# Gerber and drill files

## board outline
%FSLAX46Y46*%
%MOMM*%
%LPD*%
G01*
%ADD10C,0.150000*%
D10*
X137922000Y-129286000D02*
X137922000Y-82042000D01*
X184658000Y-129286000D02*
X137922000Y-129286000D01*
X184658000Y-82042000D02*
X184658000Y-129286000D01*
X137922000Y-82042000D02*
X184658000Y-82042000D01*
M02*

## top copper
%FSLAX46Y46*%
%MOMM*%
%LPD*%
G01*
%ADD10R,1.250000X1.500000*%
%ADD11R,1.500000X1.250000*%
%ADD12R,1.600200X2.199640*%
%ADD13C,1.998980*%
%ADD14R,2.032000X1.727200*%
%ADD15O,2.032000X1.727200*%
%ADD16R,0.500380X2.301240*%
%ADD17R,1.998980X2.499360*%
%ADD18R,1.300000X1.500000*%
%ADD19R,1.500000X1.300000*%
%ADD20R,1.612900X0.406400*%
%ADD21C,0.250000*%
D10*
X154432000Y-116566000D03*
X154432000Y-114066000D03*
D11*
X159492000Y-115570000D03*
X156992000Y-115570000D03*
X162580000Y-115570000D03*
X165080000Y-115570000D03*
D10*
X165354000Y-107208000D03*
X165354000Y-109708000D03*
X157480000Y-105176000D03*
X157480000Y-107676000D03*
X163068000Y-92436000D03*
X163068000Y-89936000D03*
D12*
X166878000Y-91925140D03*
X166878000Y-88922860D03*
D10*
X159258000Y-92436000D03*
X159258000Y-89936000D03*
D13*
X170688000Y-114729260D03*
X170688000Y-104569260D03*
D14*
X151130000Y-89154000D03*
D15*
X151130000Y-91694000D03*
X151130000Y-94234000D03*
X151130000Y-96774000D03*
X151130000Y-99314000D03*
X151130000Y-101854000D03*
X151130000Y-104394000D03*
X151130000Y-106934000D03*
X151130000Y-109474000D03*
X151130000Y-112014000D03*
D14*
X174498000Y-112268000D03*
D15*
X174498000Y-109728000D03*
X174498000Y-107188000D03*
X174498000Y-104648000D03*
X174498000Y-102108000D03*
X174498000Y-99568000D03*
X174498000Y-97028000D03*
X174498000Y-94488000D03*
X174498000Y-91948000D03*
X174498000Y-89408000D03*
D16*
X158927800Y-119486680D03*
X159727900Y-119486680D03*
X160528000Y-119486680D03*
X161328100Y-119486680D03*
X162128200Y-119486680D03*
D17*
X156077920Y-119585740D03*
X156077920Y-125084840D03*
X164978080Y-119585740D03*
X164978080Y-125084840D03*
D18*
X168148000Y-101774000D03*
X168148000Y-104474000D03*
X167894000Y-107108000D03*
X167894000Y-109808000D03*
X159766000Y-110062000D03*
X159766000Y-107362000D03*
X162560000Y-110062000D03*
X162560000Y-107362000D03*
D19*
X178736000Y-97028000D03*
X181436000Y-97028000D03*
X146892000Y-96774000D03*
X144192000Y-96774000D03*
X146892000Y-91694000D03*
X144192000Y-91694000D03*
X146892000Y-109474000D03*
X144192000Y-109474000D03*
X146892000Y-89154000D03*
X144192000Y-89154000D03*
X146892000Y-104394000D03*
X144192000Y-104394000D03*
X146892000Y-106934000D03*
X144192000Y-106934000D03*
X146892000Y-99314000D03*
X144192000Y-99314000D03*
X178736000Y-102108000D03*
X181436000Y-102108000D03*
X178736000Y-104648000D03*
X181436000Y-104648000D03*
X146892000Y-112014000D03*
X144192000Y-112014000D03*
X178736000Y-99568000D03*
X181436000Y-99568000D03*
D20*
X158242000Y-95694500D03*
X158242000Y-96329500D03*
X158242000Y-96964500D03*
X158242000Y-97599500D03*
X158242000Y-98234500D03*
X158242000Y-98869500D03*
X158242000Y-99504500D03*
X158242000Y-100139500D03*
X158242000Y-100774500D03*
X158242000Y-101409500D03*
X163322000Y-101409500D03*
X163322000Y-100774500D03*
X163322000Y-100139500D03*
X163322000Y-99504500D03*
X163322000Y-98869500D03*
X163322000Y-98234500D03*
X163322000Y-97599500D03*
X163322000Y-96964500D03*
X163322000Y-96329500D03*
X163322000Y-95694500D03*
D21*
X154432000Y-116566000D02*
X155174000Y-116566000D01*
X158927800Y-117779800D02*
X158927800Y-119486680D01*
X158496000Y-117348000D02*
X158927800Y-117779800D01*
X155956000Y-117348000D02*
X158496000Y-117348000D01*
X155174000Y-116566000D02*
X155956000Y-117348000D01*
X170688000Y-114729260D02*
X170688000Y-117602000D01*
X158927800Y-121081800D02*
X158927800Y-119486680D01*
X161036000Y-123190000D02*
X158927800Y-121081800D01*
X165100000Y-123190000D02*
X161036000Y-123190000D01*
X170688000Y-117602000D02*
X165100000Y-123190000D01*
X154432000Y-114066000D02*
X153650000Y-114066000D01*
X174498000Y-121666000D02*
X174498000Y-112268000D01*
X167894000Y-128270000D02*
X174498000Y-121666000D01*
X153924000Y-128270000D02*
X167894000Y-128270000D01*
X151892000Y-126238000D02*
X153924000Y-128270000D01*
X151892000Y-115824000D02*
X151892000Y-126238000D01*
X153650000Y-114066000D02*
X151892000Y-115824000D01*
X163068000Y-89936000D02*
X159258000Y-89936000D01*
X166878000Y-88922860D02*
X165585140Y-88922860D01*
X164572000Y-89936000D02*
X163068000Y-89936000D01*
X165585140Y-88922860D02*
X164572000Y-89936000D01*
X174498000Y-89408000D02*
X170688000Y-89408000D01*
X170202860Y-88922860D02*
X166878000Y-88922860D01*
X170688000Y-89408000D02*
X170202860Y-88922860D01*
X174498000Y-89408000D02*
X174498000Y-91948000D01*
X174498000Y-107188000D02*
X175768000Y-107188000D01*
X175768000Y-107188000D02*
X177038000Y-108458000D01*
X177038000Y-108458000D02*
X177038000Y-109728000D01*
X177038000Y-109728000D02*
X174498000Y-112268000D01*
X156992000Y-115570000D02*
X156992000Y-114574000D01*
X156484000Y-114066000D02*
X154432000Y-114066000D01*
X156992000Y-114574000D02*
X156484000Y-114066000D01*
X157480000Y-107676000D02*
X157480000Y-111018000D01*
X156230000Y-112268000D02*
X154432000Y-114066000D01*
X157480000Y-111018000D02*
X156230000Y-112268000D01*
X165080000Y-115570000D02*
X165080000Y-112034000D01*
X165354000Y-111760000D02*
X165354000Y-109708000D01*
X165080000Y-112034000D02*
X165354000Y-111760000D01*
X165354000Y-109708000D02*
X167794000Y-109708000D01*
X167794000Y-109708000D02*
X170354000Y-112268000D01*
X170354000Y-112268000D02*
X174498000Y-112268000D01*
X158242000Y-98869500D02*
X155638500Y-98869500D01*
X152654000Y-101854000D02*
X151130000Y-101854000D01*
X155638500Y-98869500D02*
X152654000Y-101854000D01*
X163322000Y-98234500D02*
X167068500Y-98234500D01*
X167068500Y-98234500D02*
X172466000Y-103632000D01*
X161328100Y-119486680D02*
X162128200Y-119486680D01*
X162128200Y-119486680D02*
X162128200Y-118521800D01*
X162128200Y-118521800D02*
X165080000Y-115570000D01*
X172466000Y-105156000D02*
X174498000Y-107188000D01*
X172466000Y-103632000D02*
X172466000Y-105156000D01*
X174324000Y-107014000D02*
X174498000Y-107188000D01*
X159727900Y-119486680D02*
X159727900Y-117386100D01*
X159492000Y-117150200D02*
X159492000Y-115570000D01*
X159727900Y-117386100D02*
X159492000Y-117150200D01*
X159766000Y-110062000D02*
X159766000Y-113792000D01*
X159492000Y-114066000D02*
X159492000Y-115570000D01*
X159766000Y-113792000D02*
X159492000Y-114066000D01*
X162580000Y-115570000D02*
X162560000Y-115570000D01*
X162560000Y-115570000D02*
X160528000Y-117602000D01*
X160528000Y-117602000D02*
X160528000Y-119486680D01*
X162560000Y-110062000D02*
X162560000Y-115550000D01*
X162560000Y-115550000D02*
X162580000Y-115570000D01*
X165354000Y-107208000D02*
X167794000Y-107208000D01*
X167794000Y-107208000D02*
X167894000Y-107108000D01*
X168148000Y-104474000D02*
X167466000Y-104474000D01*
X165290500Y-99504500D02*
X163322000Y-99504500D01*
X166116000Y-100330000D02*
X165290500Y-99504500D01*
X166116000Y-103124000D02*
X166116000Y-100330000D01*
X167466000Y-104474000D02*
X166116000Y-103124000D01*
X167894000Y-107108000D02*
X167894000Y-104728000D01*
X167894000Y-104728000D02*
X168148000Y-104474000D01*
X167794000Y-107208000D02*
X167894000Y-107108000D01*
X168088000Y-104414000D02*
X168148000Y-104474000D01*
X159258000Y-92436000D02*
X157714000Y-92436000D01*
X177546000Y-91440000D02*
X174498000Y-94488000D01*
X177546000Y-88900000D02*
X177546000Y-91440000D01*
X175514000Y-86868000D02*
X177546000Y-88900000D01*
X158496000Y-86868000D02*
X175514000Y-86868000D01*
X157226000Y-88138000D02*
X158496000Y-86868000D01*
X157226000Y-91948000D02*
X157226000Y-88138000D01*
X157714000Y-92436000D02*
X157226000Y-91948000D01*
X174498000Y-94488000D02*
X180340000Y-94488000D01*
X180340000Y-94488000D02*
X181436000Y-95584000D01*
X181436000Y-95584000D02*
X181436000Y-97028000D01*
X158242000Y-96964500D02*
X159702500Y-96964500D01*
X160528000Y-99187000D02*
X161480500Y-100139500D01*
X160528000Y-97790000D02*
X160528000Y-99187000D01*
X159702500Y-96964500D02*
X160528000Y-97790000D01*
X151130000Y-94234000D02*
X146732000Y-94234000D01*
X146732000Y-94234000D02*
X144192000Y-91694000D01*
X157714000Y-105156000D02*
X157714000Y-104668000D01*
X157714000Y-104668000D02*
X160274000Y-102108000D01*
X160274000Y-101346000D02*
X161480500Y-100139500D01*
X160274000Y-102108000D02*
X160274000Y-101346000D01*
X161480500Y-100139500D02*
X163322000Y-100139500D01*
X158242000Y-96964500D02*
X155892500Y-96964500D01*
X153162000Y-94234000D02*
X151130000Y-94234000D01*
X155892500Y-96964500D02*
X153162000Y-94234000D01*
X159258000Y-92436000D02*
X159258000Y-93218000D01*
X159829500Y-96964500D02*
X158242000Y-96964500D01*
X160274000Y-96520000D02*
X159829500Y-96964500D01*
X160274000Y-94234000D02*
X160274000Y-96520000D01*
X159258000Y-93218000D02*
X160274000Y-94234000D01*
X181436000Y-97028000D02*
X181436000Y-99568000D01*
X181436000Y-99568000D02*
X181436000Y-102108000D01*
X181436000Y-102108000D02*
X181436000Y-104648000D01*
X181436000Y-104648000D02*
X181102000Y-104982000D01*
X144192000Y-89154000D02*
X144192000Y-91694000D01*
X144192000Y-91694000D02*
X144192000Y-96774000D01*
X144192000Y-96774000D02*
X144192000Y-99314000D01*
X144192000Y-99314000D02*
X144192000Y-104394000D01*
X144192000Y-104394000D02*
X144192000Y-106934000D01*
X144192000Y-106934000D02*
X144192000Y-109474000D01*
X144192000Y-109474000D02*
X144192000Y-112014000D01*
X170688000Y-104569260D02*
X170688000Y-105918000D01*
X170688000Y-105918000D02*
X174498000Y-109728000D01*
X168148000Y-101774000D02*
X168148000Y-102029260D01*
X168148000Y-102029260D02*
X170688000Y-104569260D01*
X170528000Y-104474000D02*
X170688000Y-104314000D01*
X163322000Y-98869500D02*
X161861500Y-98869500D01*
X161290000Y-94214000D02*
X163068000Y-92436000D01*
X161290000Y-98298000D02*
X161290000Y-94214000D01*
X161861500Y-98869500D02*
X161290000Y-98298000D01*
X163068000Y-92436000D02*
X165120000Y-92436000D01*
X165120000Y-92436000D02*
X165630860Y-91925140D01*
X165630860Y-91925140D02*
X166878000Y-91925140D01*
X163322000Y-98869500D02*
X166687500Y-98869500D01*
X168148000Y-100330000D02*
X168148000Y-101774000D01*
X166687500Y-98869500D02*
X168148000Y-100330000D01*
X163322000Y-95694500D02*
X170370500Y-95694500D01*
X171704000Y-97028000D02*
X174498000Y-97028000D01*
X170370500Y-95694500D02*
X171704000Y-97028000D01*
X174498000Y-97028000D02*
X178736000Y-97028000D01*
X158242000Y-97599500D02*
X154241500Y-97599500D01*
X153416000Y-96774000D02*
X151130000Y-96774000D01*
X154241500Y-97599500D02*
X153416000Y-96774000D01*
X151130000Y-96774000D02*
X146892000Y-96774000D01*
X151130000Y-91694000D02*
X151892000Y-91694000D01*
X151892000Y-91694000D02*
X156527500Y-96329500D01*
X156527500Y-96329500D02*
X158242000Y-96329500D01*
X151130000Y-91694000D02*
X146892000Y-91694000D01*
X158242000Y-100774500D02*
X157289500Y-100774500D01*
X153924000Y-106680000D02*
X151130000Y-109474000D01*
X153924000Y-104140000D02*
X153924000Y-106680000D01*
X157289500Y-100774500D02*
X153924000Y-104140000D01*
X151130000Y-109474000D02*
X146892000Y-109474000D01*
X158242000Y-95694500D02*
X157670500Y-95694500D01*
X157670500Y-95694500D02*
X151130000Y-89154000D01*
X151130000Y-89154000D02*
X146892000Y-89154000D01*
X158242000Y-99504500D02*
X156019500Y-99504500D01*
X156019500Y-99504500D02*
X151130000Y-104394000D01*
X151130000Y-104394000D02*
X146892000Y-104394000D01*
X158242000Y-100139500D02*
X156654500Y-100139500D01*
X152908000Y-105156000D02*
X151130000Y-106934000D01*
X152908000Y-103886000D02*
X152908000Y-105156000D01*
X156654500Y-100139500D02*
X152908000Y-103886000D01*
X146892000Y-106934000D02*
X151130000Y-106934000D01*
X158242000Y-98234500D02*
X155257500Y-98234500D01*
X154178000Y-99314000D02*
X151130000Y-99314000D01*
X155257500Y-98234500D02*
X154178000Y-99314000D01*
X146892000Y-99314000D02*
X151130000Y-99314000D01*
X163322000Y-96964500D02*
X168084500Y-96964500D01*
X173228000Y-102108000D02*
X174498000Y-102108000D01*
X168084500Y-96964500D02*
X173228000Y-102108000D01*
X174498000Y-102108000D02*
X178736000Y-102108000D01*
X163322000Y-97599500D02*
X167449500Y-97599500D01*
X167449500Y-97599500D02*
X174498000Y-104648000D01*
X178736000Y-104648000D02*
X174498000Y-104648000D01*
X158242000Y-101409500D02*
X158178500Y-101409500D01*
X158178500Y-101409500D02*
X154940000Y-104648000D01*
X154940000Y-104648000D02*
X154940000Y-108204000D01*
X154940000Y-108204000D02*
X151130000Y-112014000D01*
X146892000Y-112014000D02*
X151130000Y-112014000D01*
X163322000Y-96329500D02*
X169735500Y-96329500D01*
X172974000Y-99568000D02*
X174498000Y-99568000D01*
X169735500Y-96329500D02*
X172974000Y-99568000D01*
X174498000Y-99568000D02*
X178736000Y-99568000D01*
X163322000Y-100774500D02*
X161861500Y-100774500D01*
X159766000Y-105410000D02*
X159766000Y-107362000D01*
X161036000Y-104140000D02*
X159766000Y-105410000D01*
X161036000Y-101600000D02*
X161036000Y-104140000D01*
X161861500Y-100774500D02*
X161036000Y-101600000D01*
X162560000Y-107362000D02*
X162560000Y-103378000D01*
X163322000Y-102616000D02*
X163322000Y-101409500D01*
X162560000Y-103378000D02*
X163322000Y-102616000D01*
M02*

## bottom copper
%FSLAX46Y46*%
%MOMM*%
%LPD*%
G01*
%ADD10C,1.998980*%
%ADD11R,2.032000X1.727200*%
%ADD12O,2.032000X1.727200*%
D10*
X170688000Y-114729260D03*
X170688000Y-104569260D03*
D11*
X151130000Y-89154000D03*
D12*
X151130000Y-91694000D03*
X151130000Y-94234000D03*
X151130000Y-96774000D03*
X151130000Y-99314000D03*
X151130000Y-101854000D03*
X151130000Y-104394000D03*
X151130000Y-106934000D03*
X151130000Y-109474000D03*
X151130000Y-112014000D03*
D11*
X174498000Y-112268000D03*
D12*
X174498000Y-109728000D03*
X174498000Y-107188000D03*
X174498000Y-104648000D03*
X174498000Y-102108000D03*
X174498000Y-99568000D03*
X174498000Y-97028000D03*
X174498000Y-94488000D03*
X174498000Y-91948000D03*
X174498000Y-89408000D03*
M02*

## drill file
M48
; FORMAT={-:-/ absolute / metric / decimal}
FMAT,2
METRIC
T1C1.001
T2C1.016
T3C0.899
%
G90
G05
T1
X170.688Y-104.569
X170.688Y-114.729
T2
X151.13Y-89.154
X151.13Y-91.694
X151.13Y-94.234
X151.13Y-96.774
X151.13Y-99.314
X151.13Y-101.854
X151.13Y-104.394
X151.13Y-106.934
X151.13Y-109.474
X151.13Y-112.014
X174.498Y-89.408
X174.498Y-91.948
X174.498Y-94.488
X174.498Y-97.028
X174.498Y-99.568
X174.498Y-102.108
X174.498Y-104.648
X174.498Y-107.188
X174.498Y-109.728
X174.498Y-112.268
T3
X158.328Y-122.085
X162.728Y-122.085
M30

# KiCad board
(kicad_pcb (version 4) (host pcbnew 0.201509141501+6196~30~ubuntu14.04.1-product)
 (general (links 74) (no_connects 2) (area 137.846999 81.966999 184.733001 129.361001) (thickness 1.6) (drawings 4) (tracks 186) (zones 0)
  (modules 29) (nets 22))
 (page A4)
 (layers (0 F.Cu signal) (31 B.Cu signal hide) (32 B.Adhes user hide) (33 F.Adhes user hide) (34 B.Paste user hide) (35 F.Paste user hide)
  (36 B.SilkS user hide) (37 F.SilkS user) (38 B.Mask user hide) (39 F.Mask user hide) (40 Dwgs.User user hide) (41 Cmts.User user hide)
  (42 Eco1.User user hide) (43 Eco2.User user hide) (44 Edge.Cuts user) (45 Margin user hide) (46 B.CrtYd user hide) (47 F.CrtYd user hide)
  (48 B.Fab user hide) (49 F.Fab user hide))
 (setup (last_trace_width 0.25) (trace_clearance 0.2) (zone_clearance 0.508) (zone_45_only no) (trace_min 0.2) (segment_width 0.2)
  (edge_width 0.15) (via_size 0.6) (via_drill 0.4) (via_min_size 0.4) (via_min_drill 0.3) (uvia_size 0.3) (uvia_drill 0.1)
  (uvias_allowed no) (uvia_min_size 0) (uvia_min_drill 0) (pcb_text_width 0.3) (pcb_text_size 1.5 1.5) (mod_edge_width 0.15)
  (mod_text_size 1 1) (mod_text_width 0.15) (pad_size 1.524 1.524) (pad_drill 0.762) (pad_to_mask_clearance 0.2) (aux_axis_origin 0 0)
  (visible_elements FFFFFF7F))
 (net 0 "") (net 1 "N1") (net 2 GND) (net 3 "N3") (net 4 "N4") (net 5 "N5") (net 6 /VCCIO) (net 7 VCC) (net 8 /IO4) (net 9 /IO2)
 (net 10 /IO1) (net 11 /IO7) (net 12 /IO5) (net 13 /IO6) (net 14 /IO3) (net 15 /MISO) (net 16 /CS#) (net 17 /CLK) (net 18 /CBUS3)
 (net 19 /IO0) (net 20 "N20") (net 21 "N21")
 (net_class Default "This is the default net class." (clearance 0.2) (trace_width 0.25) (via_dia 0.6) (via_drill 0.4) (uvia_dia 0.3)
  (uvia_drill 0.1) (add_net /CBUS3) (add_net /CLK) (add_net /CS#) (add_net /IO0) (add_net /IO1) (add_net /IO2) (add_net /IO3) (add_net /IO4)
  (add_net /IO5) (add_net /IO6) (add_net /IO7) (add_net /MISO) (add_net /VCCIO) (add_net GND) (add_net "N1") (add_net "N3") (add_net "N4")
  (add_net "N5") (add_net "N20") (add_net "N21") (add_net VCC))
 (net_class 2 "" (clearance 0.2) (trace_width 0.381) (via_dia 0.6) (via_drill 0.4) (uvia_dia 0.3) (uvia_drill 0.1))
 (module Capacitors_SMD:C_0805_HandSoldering (layer F.Cu) (at 154.432 115.316 90)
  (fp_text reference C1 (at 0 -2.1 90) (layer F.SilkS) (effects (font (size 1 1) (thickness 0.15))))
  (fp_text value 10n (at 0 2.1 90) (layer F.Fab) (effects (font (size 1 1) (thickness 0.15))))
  (pad 1 smd rect (at -1.25 0 90) (size 1.5 1.25) (layers F.Cu F.Paste F.Mask) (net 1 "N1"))
  (pad 2 smd rect (at 1.25 0 90) (size 1.5 1.25) (layers F.Cu F.Paste F.Mask) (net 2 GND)))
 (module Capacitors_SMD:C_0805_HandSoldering (layer F.Cu) (at 158.242 115.57 180)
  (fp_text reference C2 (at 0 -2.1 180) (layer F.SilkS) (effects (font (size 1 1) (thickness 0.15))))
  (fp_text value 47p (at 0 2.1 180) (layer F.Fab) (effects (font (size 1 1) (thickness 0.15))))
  (pad 1 smd rect (at -1.25 0 180) (size 1.5 1.25) (layers F.Cu F.Paste F.Mask) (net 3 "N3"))
  (pad 2 smd rect (at 1.25 0 180) (size 1.5 1.25) (layers F.Cu F.Paste F.Mask) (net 2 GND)))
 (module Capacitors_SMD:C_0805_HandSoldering (layer F.Cu) (at 163.83 115.57)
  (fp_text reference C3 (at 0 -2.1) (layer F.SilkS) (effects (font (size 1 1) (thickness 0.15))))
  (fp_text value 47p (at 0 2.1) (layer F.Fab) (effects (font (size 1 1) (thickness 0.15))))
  (pad 1 smd rect (at -1.25 0) (size 1.5 1.25) (layers F.Cu F.Paste F.Mask) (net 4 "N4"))
  (pad 2 smd rect (at 1.25 0) (size 1.5 1.25) (layers F.Cu F.Paste F.Mask) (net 2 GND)))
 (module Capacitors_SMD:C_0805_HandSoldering (layer F.Cu) (at 165.354 108.458 270)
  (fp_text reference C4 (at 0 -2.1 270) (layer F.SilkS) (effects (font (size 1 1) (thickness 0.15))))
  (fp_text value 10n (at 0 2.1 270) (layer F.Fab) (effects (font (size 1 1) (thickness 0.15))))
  (pad 1 smd rect (at -1.25 0 270) (size 1.5 1.25) (layers F.Cu F.Paste F.Mask) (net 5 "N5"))
  (pad 2 smd rect (at 1.25 0 270) (size 1.5 1.25) (layers F.Cu F.Paste F.Mask) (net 2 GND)))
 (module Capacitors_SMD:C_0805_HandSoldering (layer F.Cu) (at 157.48 106.426 270)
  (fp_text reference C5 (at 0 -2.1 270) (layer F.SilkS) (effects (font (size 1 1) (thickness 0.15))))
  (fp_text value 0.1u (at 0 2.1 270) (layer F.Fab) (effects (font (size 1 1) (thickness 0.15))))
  (pad 1 smd rect (at -1.25 0 270) (size 1.5 1.25) (layers F.Cu F.Paste F.Mask) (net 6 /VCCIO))
  (pad 2 smd rect (at 1.25 0 270) (size 1.5 1.25) (layers F.Cu F.Paste F.Mask) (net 2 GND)))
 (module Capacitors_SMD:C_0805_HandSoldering (layer F.Cu) (at 163.068 91.186 90)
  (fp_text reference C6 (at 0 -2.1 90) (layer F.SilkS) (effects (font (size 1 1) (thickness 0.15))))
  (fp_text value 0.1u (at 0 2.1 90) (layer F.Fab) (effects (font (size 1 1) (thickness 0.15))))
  (pad 1 smd rect (at -1.25 0 90) (size 1.5 1.25) (layers F.Cu F.Paste F.Mask) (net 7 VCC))
  (pad 2 smd rect (at 1.25 0 90) (size 1.5 1.25) (layers F.Cu F.Paste F.Mask) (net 2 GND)))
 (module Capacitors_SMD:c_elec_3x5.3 (layer F.Cu) (at 166.878 90.424 270)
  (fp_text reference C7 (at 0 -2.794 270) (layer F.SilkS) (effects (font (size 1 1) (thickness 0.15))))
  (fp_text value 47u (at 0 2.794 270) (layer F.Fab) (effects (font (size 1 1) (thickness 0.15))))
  (pad 1 smd rect (at 1.50114 0 270) (size 2.19964 1.6002) (layers F.Cu F.Paste F.Mask) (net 7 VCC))
  (pad 2 smd rect (at -1.50114 0 270) (size 2.19964 1.6002) (layers F.Cu F.Paste F.Mask) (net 2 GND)))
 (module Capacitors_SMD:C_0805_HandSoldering (layer F.Cu) (at 159.258 91.186 90)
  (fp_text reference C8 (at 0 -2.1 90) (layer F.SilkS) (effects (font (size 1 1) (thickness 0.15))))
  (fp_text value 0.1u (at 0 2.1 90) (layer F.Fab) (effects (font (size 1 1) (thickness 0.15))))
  (pad 1 smd rect (at -1.25 0 90) (size 1.5 1.25) (layers F.Cu F.Paste F.Mask) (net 6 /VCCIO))
  (pad 2 smd rect (at 1.25 0 90) (size 1.5 1.25) (layers F.Cu F.Paste F.Mask) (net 2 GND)))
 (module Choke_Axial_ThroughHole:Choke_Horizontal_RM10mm (layer F.Cu) (at 170.688 109.728 90)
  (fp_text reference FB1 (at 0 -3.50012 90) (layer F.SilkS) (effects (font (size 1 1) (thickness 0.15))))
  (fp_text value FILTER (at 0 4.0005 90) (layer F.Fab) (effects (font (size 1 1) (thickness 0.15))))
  (pad 1 thru_hole circle (at -5.00126 0 90) (size 1.99898 1.99898) (drill 1.00076) (layers *.Cu *.Mask F.SilkS) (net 1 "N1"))
  (pad 2 thru_hole circle (at 5.15874 0 90) (size 1.99898 1.99898) (drill 1.00076) (layers *.Cu *.Mask F.SilkS) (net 7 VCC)))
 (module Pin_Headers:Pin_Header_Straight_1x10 (layer F.Cu) (at 151.13 89.154)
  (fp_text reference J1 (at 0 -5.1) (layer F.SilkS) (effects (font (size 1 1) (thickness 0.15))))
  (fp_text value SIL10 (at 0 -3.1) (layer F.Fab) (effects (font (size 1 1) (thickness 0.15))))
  (pad 1 thru_hole rect (at 0 0) (size 2.032 1.7272) (drill 1.016) (layers *.Cu *.Mask F.SilkS) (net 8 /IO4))
  (pad 2 thru_hole oval (at 0 2.54) (size 2.032 1.7272) (drill 1.016) (layers *.Cu *.Mask F.SilkS) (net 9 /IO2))
  (pad 3 thru_hole oval (at 0 5.08) (size 2.032 1.7272) (drill 1.016) (layers *.Cu *.Mask F.SilkS) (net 6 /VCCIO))
  (pad 4 thru_hole oval (at 0 7.62) (size 2.032 1.7272) (drill 1.016) (layers *.Cu *.Mask F.SilkS) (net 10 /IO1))
  (pad 5 thru_hole oval (at 0 10.16) (size 2.032 1.7272) (drill 1.016) (layers *.Cu *.Mask F.SilkS) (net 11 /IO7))
  (pad 6 thru_hole oval (at 0 12.7) (size 2.032 1.7272) (drill 1.016) (layers *.Cu *.Mask F.SilkS) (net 2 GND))
  (pad 7 thru_hole oval (at 0 15.24) (size 2.032 1.7272) (drill 1.016) (layers *.Cu *.Mask F.SilkS) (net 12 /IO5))
  (pad 8 thru_hole oval (at 0 17.78) (size 2.032 1.7272) (drill 1.016) (layers *.Cu *.Mask F.SilkS) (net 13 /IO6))
  (pad 9 thru_hole oval (at 0 20.32) (size 2.032 1.7272) (drill 1.016) (layers *.Cu *.Mask F.SilkS) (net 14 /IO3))
  (pad 10 thru_hole oval (at 0 22.86) (size 2.032 1.7272) (drill 1.016) (layers *.Cu *.Mask F.SilkS) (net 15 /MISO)))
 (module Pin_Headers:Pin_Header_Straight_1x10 (layer F.Cu) (at 174.498 112.268 180)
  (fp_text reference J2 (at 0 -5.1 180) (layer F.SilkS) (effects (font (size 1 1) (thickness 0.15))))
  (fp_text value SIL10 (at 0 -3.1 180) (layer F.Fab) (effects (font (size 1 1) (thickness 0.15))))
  (pad 1 thru_hole rect (at 0 0 180) (size 2.032 1.7272) (drill 1.016) (layers *.Cu *.Mask F.SilkS) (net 2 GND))
  (pad 2 thru_hole oval (at 0 2.54 180) (size 2.032 1.7272) (drill 1.016) (layers *.Cu *.Mask F.SilkS) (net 7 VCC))
  (pad 3 thru_hole oval (at 0 5.08 180) (size 2.032 1.7272) (drill 1.016) (layers *.Cu *.Mask F.SilkS) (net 2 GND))
  (pad 4 thru_hole oval (at 0 7.62 180) (size 2.032 1.7272) (drill 1.016) (layers *.Cu *.Mask F.SilkS) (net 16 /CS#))
  (pad 5 thru_hole oval (at 0 10.16 180) (size 2.032 1.7272) (drill 1.016) (layers *.Cu *.Mask F.SilkS) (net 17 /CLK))
  (pad 6 thru_hole oval (at 0 12.7 180) (size 2.032 1.7272) (drill 1.016) (layers *.Cu *.Mask F.SilkS) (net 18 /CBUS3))
  (pad 7 thru_hole oval (at 0 15.24 180) (size 2.032 1.7272) (drill 1.016) (layers *.Cu *.Mask F.SilkS) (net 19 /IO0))
  (pad 8 thru_hole oval (at 0 17.78 180) (size 2.032 1.7272) (drill 1.016) (layers *.Cu *.Mask F.SilkS) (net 6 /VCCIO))
  (pad 9 thru_hole oval (at 0 20.32 180) (size 2.032 1.7272) (drill 1.016) (layers *.Cu *.Mask F.SilkS) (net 2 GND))
  (pad 10 thru_hole oval (at 0 22.86 180) (size 2.032 1.7272) (drill 1.016) (layers *.Cu *.Mask F.SilkS) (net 2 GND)))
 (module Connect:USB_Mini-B (layer F.Cu) (at 160.528 122.936 90)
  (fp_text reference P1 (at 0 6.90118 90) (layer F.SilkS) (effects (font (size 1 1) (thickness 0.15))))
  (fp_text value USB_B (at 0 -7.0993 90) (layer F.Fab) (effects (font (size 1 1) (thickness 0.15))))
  (pad 1 smd rect (at 3.44932 -1.6002 90) (size 2.30124 0.50038) (layers F.Cu F.Paste F.Mask) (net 1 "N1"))
  (pad 2 smd rect (at 3.44932 -0.8001 90) (size 2.30124 0.50038) (layers F.Cu F.Paste F.Mask) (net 3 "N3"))
  (pad 3 smd rect (at 3.44932 0 90) (size 2.30124 0.50038) (layers F.Cu F.Paste F.Mask) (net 4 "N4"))
  (pad 4 smd rect (at 3.44932 0.8001 90) (size 2.30124 0.50038) (layers F.Cu F.Paste F.Mask) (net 2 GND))
  (pad 5 smd rect (at 3.44932 1.6002 90) (size 2.30124 0.50038) (layers F.Cu F.Paste F.Mask) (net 2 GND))
  (pad 6 smd rect (at 3.35026 -4.45008 90) (size 2.49936 1.99898) (layers F.Cu F.Paste F.Mask))
  (pad 6 smd rect (at -2.14884 -4.45008 90) (size 2.49936 1.99898) (layers F.Cu F.Paste F.Mask))
  (pad 6 smd rect (at 3.35026 4.45008 90) (size 2.49936 1.99898) (layers F.Cu F.Paste F.Mask))
  (pad 6 smd rect (at -2.14884 4.45008 90) (size 2.49936 1.99898) (layers F.Cu F.Paste F.Mask))
  (pad "" np_thru_hole circle (at 0.8509 -2.19964 90) (size 0.89916 0.89916) (drill 0.89916) (layers *.Cu *.Mask F.SilkS))
  (pad "" np_thru_hole circle (at 0.8509 2.19964 90) (size 0.89916 0.89916) (drill 0.89916) (layers *.Cu *.Mask F.SilkS)))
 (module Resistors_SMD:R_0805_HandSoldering (layer F.Cu) (at 168.148 103.124 270)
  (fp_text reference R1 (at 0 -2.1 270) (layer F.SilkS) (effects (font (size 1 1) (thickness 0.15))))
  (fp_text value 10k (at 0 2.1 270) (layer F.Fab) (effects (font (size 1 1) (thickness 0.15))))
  (pad 1 smd rect (at -1.35 0 270) (size 1.5 1.3) (layers F.Cu F.Paste F.Mask) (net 7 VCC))
  (pad 2 smd rect (at 1.35 0 270) (size 1.5 1.3) (layers F.Cu F.Paste F.Mask) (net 5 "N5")))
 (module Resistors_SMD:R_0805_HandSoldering (layer F.Cu) (at 167.894 108.458 270)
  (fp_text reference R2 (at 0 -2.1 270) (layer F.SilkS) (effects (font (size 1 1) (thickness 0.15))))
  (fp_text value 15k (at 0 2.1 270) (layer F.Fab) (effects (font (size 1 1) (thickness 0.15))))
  (pad 1 smd rect (at -1.35 0 270) (size 1.5 1.3) (layers F.Cu F.Paste F.Mask) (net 5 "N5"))
  (pad 2 smd rect (at 1.35 0 270) (size 1.5 1.3) (layers F.Cu F.Paste F.Mask) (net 2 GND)))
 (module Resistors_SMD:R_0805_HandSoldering (layer F.Cu) (at 159.766 108.712 90)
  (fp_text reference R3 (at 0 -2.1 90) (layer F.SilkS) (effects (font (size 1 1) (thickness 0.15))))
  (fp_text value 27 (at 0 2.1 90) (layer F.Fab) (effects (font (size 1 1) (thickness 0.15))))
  (pad 1 smd rect (at -1.35 0 90) (size 1.5 1.3) (layers F.Cu F.Paste F.Mask) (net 3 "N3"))
  (pad 2 smd rect (at 1.35 0 90) (size 1.5 1.3) (layers F.Cu F.Paste F.Mask) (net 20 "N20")))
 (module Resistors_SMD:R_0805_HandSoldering (layer F.Cu) (at 162.56 108.712 90)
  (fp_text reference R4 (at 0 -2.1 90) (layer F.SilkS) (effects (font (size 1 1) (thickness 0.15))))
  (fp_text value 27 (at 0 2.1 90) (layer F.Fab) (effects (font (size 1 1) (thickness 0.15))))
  (pad 1 smd rect (at -1.35 0 90) (size 1.5 1.3) (layers F.Cu F.Paste F.Mask) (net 4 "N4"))
  (pad 2 smd rect (at 1.35 0 90) (size 1.5 1.3) (layers F.Cu F.Paste F.Mask) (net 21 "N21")))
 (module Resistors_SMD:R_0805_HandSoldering (layer F.Cu) (at 180.086 97.028)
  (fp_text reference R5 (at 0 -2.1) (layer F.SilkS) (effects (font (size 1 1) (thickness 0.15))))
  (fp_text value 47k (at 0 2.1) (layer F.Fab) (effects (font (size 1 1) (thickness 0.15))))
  (pad 1 smd rect (at -1.35 0) (size 1.5 1.3) (layers F.Cu F.Paste F.Mask) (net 19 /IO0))
  (pad 2 smd rect (at 1.35 0) (size 1.5 1.3) (layers F.Cu F.Paste F.Mask) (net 6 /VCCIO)))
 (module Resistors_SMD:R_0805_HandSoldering (layer F.Cu) (at 145.542 96.774 180)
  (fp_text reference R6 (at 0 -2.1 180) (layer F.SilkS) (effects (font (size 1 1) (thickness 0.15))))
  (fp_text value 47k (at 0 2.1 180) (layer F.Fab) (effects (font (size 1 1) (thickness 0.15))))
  (pad 1 smd rect (at -1.35 0 180) (size 1.5 1.3) (layers F.Cu F.Paste F.Mask) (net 10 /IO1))
  (pad 2 smd rect (at 1.35 0 180) (size 1.5 1.3) (layers F.Cu F.Paste F.Mask) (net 6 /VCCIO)))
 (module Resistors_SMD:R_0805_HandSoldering (layer F.Cu) (at 145.542 91.694 180)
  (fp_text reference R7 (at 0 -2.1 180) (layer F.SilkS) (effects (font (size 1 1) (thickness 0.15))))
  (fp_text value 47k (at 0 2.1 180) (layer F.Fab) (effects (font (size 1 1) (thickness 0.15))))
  (pad 1 smd rect (at -1.35 0 180) (size 1.5 1.3) (layers F.Cu F.Paste F.Mask) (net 9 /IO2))
  (pad 2 smd rect (at 1.35 0 180) (size 1.5 1.3) (layers F.Cu F.Paste F.Mask) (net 6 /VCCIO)))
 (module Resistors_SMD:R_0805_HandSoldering (layer F.Cu) (at 145.542 109.474 180)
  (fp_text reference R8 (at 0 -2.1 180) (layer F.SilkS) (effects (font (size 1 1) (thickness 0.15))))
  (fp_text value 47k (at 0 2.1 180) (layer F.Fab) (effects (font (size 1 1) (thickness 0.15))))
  (pad 1 smd rect (at -1.35 0 180) (size 1.5 1.3) (layers F.Cu F.Paste F.Mask) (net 14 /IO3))
  (pad 2 smd rect (at 1.35 0 180) (size 1.5 1.3) (layers F.Cu F.Paste F.Mask) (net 6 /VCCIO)))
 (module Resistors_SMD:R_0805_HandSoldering (layer F.Cu) (at 145.542 89.154 180)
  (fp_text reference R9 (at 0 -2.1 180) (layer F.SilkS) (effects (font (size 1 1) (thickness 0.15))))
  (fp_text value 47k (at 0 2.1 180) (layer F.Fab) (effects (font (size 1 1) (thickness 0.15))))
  (pad 1 smd rect (at -1.35 0 180) (size 1.5 1.3) (layers F.Cu F.Paste F.Mask) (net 8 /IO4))
  (pad 2 smd rect (at 1.35 0 180) (size 1.5 1.3) (layers F.Cu F.Paste F.Mask) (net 6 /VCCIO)))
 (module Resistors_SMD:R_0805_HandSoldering (layer F.Cu) (at 145.542 104.394 180)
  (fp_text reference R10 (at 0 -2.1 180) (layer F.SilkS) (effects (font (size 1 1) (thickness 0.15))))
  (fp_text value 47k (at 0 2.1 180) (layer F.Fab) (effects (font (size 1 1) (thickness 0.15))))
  (pad 1 smd rect (at -1.35 0 180) (size 1.5 1.3) (layers F.Cu F.Paste F.Mask) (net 12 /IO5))
  (pad 2 smd rect (at 1.35 0 180) (size 1.5 1.3) (layers F.Cu F.Paste F.Mask) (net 6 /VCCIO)))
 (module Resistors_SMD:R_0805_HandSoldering (layer F.Cu) (at 145.542 106.934 180)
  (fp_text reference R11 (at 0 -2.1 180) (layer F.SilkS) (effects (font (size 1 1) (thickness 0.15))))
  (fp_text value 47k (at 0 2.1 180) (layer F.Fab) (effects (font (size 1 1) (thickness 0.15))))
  (pad 1 smd rect (at -1.35 0 180) (size 1.5 1.3) (layers F.Cu F.Paste F.Mask) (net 13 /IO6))
  (pad 2 smd rect (at 1.35 0 180) (size 1.5 1.3) (layers F.Cu F.Paste F.Mask) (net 6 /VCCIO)))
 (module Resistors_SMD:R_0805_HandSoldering (layer F.Cu) (at 145.542 99.314 180)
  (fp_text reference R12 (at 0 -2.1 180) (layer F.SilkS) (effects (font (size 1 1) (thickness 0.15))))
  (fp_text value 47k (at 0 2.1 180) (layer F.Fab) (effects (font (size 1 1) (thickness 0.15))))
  (pad 1 smd rect (at -1.35 0 180) (size 1.5 1.3) (layers F.Cu F.Paste F.Mask) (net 11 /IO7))
  (pad 2 smd rect (at 1.35 0 180) (size 1.5 1.3) (layers F.Cu F.Paste F.Mask) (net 6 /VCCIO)))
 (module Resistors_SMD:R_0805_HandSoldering (layer F.Cu) (at 180.086 102.108)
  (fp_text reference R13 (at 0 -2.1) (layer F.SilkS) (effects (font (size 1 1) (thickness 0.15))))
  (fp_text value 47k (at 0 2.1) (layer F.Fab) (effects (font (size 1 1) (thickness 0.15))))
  (pad 1 smd rect (at -1.35 0) (size 1.5 1.3) (layers F.Cu F.Paste F.Mask) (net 17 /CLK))
  (pad 2 smd rect (at 1.35 0) (size 1.5 1.3) (layers F.Cu F.Paste F.Mask) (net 6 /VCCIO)))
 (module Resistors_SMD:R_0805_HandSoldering (layer F.Cu) (at 180.086 104.648)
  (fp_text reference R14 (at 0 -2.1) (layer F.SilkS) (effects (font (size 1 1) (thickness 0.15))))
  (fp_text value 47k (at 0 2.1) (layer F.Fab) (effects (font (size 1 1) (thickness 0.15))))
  (pad 1 smd rect (at -1.35 0) (size 1.5 1.3) (layers F.Cu F.Paste F.Mask) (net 16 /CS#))
  (pad 2 smd rect (at 1.35 0) (size 1.5 1.3) (layers F.Cu F.Paste F.Mask) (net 6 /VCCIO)))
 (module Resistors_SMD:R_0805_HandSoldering (layer F.Cu) (at 145.542 112.014 180)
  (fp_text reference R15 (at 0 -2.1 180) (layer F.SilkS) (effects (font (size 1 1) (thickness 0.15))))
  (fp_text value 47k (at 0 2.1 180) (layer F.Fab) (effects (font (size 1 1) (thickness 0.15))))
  (pad 1 smd rect (at -1.35 0 180) (size 1.5 1.3) (layers F.Cu F.Paste F.Mask) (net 15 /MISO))
  (pad 2 smd rect (at 1.35 0 180) (size 1.5 1.3) (layers F.Cu F.Paste F.Mask) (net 6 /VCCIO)))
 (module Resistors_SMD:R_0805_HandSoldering (layer F.Cu) (at 180.086 99.568)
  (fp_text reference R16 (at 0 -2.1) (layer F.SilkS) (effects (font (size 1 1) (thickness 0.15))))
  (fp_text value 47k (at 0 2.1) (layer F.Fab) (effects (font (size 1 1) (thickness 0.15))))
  (pad 1 smd rect (at -1.35 0) (size 1.5 1.3) (layers F.Cu F.Paste F.Mask) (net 18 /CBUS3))
  (pad 2 smd rect (at 1.35 0) (size 1.5 1.3) (layers F.Cu F.Paste F.Mask) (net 6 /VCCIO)))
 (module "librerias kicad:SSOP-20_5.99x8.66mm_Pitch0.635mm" (layer F.Cu) (at 160.782 98.552)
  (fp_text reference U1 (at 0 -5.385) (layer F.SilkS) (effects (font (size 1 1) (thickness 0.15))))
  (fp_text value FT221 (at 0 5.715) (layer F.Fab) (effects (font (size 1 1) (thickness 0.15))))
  (pad 1 smd rect (at -2.54 -2.8575) (size 1.6129 0.4064) (layers F.Cu F.Paste F.Mask) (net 8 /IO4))
  (pad 2 smd rect (at -2.54 -2.2225) (size 1.6129 0.4064) (layers F.Cu F.Paste F.Mask) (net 9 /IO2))
  (pad 3 smd rect (at -2.54 -1.5875) (size 1.6129 0.4064) (layers F.Cu F.Paste F.Mask) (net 6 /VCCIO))
  (pad 4 smd rect (at -2.54 -0.9525) (size 1.6129 0.4064) (layers F.Cu F.Paste F.Mask) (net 10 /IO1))
  (pad 5 smd rect (at -2.54 -0.3175) (size 1.6129 0.4064) (layers F.Cu F.Paste F.Mask) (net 11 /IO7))
  (pad 6 smd rect (at -2.54 0.3175) (size 1.6129 0.4064) (layers F.Cu F.Paste F.Mask) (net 2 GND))
  (pad 7 smd rect (at -2.54 0.9525) (size 1.6129 0.4064) (layers F.Cu F.Paste F.Mask) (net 12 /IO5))
  (pad 8 smd rect (at -2.54 1.5875) (size 1.6129 0.4064) (layers F.Cu F.Paste F.Mask) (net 13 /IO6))
  (pad 9 smd rect (at -2.54 2.2225) (size 1.6129 0.4064) (layers F.Cu F.Paste F.Mask) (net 14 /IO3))
  (pad 10 smd rect (at -2.54 2.8575) (size 1.6129 0.4064) (layers F.Cu F.Paste F.Mask) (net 15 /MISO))
  (pad 11 smd rect (at 2.54 2.8575) (size 1.6129 0.4064) (layers F.Cu F.Paste F.Mask) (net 21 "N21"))
  (pad 12 smd rect (at 2.54 2.2225) (size 1.6129 0.4064) (layers F.Cu F.Paste F.Mask) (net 20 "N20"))
  (pad 13 smd rect (at 2.54 1.5875) (size 1.6129 0.4064) (layers F.Cu F.Paste F.Mask) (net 6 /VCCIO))
  (pad 14 smd rect (at 2.54 0.9525) (size 1.6129 0.4064) (layers F.Cu F.Paste F.Mask) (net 5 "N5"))
  (pad 15 smd rect (at 2.54 0.3175) (size 1.6129 0.4064) (layers F.Cu F.Paste F.Mask) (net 7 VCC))
  (pad 16 smd rect (at 2.54 -0.3175) (size 1.6129 0.4064) (layers F.Cu F.Paste F.Mask) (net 2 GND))
  (pad 17 smd rect (at 2.54 -0.9525) (size 1.6129 0.4064) (layers F.Cu F.Paste F.Mask) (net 16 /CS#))
  (pad 18 smd rect (at 2.54 -1.5875) (size 1.6129 0.4064) (layers F.Cu F.Paste F.Mask) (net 17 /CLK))
  (pad 19 smd rect (at 2.54 -2.2225) (size 1.6129 0.4064) (layers F.Cu F.Paste F.Mask) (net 18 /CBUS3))
  (pad 20 smd rect (at 2.54 -2.8575) (size 1.6129 0.4064) (layers F.Cu F.Paste F.Mask) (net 19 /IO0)))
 (gr_line (start 137.922 129.286) (end 137.922 82.042) (angle 90) (layer Edge.Cuts) (width 0.15))
 (gr_line (start 184.658 129.286) (end 137.922 129.286) (angle 90) (layer Edge.Cuts) (width 0.15))
 (gr_line (start 184.658 82.042) (end 184.658 129.286) (angle 90) (layer Edge.Cuts) (width 0.15))
 (gr_line (start 137.922 82.042) (end 184.658 82.042) (angle 90) (layer Edge.Cuts) (width 0.15))
 (segment (start 154.432 116.566) (end 155.174 116.566) (width 0.25) (layer F.Cu) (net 1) (status 400000))
 (segment (start 158.9278 117.7798) (end 158.9278 119.48668) (width 0.25) (layer F.Cu) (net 1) (status 800000))
 (segment (start 158.496 117.348) (end 158.9278 117.7798) (width 0.25) (layer F.Cu) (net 1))
 (segment (start 155.956 117.348) (end 158.496 117.348) (width 0.25) (layer F.Cu) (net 1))
 (segment (start 155.174 116.566) (end 155.956 117.348) (width 0.25) (layer F.Cu) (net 1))
 (segment (start 170.688 114.72926) (end 170.688 117.602) (width 0.25) (layer F.Cu) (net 1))
 (segment (start 158.9278 121.0818) (end 158.9278 119.48668) (width 0.25) (layer F.Cu) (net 1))
 (segment (start 161.036 123.19) (end 158.9278 121.0818) (width 0.25) (layer F.Cu) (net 1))
 (segment (start 165.1 123.19) (end 161.036 123.19) (width 0.25) (layer F.Cu) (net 1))
 (segment (start 170.688 117.602) (end 165.1 123.19) (width 0.25) (layer F.Cu) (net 1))
 (segment (start 154.432 114.066) (end 153.65 114.066) (width 0.25) (layer F.Cu) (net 2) (status 400000))
 (segment (start 174.498 121.666) (end 174.498 112.268) (width 0.25) (layer F.Cu) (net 2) (status 800000))
 (segment (start 167.894 128.27) (end 174.498 121.666) (width 0.25) (layer F.Cu) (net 2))
 (segment (start 153.924 128.27) (end 167.894 128.27) (width 0.25) (layer F.Cu) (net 2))
 (segment (start 151.892 126.238) (end 153.924 128.27) (width 0.25) (layer F.Cu) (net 2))
 (segment (start 151.892 115.824) (end 151.892 126.238) (width 0.25) (layer F.Cu) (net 2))
 (segment (start 153.65 114.066) (end 151.892 115.824) (width 0.25) (layer F.Cu) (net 2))
 (segment (start 163.068 89.936) (end 159.258 89.936) (width 0.25) (layer F.Cu) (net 2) (status C00000))
 (segment (start 166.878 88.92286) (end 165.58514 88.92286) (width 0.25) (layer F.Cu) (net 2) (status 400000))
 (segment (start 164.572 89.936) (end 163.068 89.936) (width 0.25) (layer F.Cu) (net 2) (status 800000))
 (segment (start 165.58514 88.92286) (end 164.572 89.936) (width 0.25) (layer F.Cu) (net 2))
 (segment (start 174.498 89.408) (end 170.688 89.408) (width 0.25) (layer F.Cu) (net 2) (status 400000))
 (segment (start 170.20286 88.92286) (end 166.878 88.92286) (width 0.25) (layer F.Cu) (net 2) (status 800000))
 (segment (start 170.688 89.408) (end 170.20286 88.92286) (width 0.25) (layer F.Cu) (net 2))
 (segment (start 174.498 89.408) (end 174.498 91.948) (width 0.25) (layer F.Cu) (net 2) (status C00000))
 (segment (start 174.498 107.188) (end 175.768 107.188) (width 0.25) (layer F.Cu) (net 2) (status 400000))
 (segment (start 175.768 107.188) (end 177.038 108.458) (width 0.25) (layer F.Cu) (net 2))
 (segment (start 177.038 108.458) (end 177.038 109.728) (width 0.25) (layer F.Cu) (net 2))
 (segment (start 177.038 109.728) (end 174.498 112.268) (width 0.25) (layer F.Cu) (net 2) (status 800000))
 (segment (start 156.992 115.57) (end 156.992 114.574) (width 0.25) (layer F.Cu) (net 2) (status 400000))
 (segment (start 156.484 114.066) (end 154.432 114.066) (width 0.25) (layer F.Cu) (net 2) (status 800000))
 (segment (start 156.992 114.574) (end 156.484 114.066) (width 0.25) (layer F.Cu) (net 2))
 (segment (start 157.48 107.676) (end 157.48 111.018) (width 0.25) (layer F.Cu) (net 2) (status 400000))
 (segment (start 156.23 112.268) (end 154.432 114.066) (width 0.25) (layer F.Cu) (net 2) (status 800000))
 (segment (start 157.48 111.018) (end 156.23 112.268) (width 0.25) (layer F.Cu) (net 2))
 (segment (start 165.08 115.57) (end 165.08 112.034) (width 0.25) (layer F.Cu) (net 2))
 (segment (start 165.354 111.76) (end 165.354 109.708) (width 0.25) (layer F.Cu) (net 2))
 (segment (start 165.08 112.034) (end 165.354 111.76) (width 0.25) (layer F.Cu) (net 2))
 (segment (start 165.354 109.708) (end 167.794 109.708) (width 0.25) (layer F.Cu) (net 2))
 (segment (start 167.794 109.708) (end 170.354 112.268) (width 0.25) (layer F.Cu) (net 2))
 (segment (start 170.354 112.268) (end 174.498 112.268) (width 0.25) (layer F.Cu) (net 2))
 (segment (start 158.242 98.8695) (end 155.6385 98.8695) (width 0.25) (layer F.Cu) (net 2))
 (segment (start 152.654 101.854) (end 151.13 101.854) (width 0.25) (layer F.Cu) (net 2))
 (segment (start 155.6385 98.8695) (end 152.654 101.854) (width 0.25) (layer F.Cu) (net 2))
 (segment (start 163.322 98.2345) (end 167.0685 98.2345) (width 0.25) (layer F.Cu) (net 2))
 (segment (start 167.0685 98.2345) (end 172.466 103.632) (width 0.25) (layer F.Cu) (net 2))
 (segment (start 161.3281 119.48668) (end 162.1282 119.48668) (width 0.25) (layer F.Cu) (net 2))
 (segment (start 162.1282 119.48668) (end 162.1282 118.5218) (width 0.25) (layer F.Cu) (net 2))
 (segment (start 162.1282 118.5218) (end 165.08 115.57) (width 0.25) (layer F.Cu) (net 2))
 (segment (start 172.466 105.156) (end 174.498 107.188) (width 0.25) (layer F.Cu) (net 2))
 (segment (start 172.466 103.632) (end 172.466 105.156) (width 0.25) (layer F.Cu) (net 2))
 (segment (start 174.324 107.014) (end 174.498 107.188) (width 0.25) (layer F.Cu) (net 2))
 (segment (start 159.7279 119.48668) (end 159.7279 117.3861) (width 0.25) (layer F.Cu) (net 3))
 (segment (start 159.492 117.1502) (end 159.492 115.57) (width 0.25) (layer F.Cu) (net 3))
 (segment (start 159.7279 117.3861) (end 159.492 117.1502) (width 0.25) (layer F.Cu) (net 3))
 (segment (start 159.766 110.062) (end 159.766 113.792) (width 0.25) (layer F.Cu) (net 3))
 (segment (start 159.492 114.066) (end 159.492 115.57) (width 0.25) (layer F.Cu) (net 3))
 (segment (start 159.766 113.792) (end 159.492 114.066) (width 0.25) (layer F.Cu) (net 3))
 (segment (start 162.58 115.57) (end 162.56 115.57) (width 0.25) (layer F.Cu) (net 4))
 (segment (start 162.56 115.57) (end 160.528 117.602) (width 0.25) (layer F.Cu) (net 4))
 (segment (start 160.528 117.602) (end 160.528 119.48668) (width 0.25) (layer F.Cu) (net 4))
 (segment (start 162.56 110.062) (end 162.56 115.55) (width 0.25) (layer F.Cu) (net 4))
 (segment (start 162.56 115.55) (end 162.58 115.57) (width 0.25) (layer F.Cu) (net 4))
 (segment (start 165.354 107.208) (end 167.794 107.208) (width 0.25) (layer F.Cu) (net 5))
 (segment (start 167.794 107.208) (end 167.894 107.108) (width 0.25) (layer F.Cu) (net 5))
 (segment (start 168.148 104.474) (end 167.466 104.474) (width 0.25) (layer F.Cu) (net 5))
 (segment (start 165.2905 99.5045) (end 163.322 99.5045) (width 0.25) (layer F.Cu) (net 5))
 (segment (start 166.116 100.33) (end 165.2905 99.5045) (width 0.25) (layer F.Cu) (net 5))
 (segment (start 166.116 103.124) (end 166.116 100.33) (width 0.25) (layer F.Cu) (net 5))
 (segment (start 167.466 104.474) (end 166.116 103.124) (width 0.25) (layer F.Cu) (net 5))
 (segment (start 167.894 107.108) (end 167.894 104.728) (width 0.25) (layer F.Cu) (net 5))
 (segment (start 167.894 104.728) (end 168.148 104.474) (width 0.25) (layer F.Cu) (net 5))
 (segment (start 167.794 107.208) (end 167.894 107.108) (width 0.25) (layer F.Cu) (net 5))
 (segment (start 168.088 104.414) (end 168.148 104.474) (width 0.25) (layer F.Cu) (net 5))
 (segment (start 159.258 92.436) (end 157.714 92.436) (width 0.25) (layer F.Cu) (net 6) (status 400000))
 (segment (start 177.546 91.44) (end 174.498 94.488) (width 0.25) (layer F.Cu) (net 6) (status 800000))
 (segment (start 177.546 88.9) (end 177.546 91.44) (width 0.25) (layer F.Cu) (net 6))
 (segment (start 175.514 86.868) (end 177.546 88.9) (width 0.25) (layer F.Cu) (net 6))
 (segment (start 158.496 86.868) (end 175.514 86.868) (width 0.25) (layer F.Cu) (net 6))
 (segment (start 157.226 88.138) (end 158.496 86.868) (width 0.25) (layer F.Cu) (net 6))
 (segment (start 157.226 91.948) (end 157.226 88.138) (width 0.25) (layer F.Cu) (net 6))
 (segment (start 157.714 92.436) (end 157.226 91.948) (width 0.25) (layer F.Cu) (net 6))
 (segment (start 174.498 94.488) (end 180.34 94.488) (width 0.25) (layer F.Cu) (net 6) (status 400000))
 (segment (start 180.34 94.488) (end 181.436 95.584) (width 0.25) (layer F.Cu) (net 6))
 (segment (start 181.436 95.584) (end 181.436 97.028) (width 0.25) (layer F.Cu) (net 6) (status 800000))
 (segment (start 158.242 96.9645) (end 159.7025 96.9645) (width 0.25) (layer F.Cu) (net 6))
 (segment (start 160.528 99.187) (end 161.4805 100.1395) (width 0.25) (layer F.Cu) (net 6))
 (segment (start 160.528 97.79) (end 160.528 99.187) (width 0.25) (layer F.Cu) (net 6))
 (segment (start 159.7025 96.9645) (end 160.528 97.79) (width 0.25) (layer F.Cu) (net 6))
 (segment (start 151.13 94.234) (end 146.732 94.234) (width 0.25) (layer F.Cu) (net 6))
 (segment (start 146.732 94.234) (end 144.192 91.694) (width 0.25) (layer F.Cu) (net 6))
 (segment (start 157.714 105.156) (end 157.714 104.668) (width 0.25) (layer F.Cu) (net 6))
 (segment (start 157.714 104.668) (end 160.274 102.108) (width 0.25) (layer F.Cu) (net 6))
 (segment (start 160.274 101.346) (end 161.4805 100.1395) (width 0.25) (layer F.Cu) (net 6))
 (segment (start 160.274 102.108) (end 160.274 101.346) (width 0.25) (layer F.Cu) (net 6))
 (segment (start 161.4805 100.1395) (end 163.322 100.1395) (width 0.25) (layer F.Cu) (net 6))
 (segment (start 158.242 96.9645) (end 155.8925 96.9645) (width 0.25) (layer F.Cu) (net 6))
 (segment (start 153.162 94.234) (end 151.13 94.234) (width 0.25) (layer F.Cu) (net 6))
 (segment (start 155.8925 96.9645) (end 153.162 94.234) (width 0.25) (layer F.Cu) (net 6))
 (segment (start 159.258 92.436) (end 159.258 93.218) (width 0.25) (layer F.Cu) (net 6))
 (segment (start 159.8295 96.9645) (end 158.242 96.9645) (width 0.25) (layer F.Cu) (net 6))
 (segment (start 160.274 96.52) (end 159.8295 96.9645) (width 0.25) (layer F.Cu) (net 6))
 (segment (start 160.274 94.234) (end 160.274 96.52) (width 0.25) (layer F.Cu) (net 6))
 (segment (start 159.258 93.218) (end 160.274 94.234) (width 0.25) (layer F.Cu) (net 6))
 (segment (start 181.436 97.028) (end 181.436 99.568) (width 0.25) (layer F.Cu) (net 6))
 (segment (start 181.436 99.568) (end 181.436 102.108) (width 0.25) (layer F.Cu) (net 6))
 (segment (start 181.436 102.108) (end 181.436 104.648) (width 0.25) (layer F.Cu) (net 6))
 (segment (start 181.436 104.648) (end 181.102 104.982) (width 0.25) (layer F.Cu) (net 6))
 (segment (start 144.192 89.154) (end 144.192 91.694) (width 0.25) (layer F.Cu) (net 6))
 (segment (start 144.192 91.694) (end 144.192 96.774) (width 0.25) (layer F.Cu) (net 6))
 (segment (start 144.192 96.774) (end 144.192 99.314) (width 0.25) (layer F.Cu) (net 6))
 (segment (start 144.192 99.314) (end 144.192 104.394) (width 0.25) (layer F.Cu) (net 6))
 (segment (start 144.192 104.394) (end 144.192 106.934) (width 0.25) (layer F.Cu) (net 6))
 (segment (start 144.192 106.934) (end 144.192 109.474) (width 0.25) (layer F.Cu) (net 6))
 (segment (start 144.192 109.474) (end 144.192 112.014) (width 0.25) (layer F.Cu) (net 6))
 (segment (start 170.688 104.56926) (end 170.688 105.918) (width 0.25) (layer F.Cu) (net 7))
 (segment (start 170.688 105.918) (end 174.498 109.728) (width 0.25) (layer F.Cu) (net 7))
 (segment (start 168.148 101.774) (end 168.148 102.02926) (width 0.25) (layer F.Cu) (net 7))
 (segment (start 168.148 102.02926) (end 170.688 104.56926) (width 0.25) (layer F.Cu) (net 7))
 (segment (start 170.528 104.474) (end 170.688 104.314) (width 0.25) (layer F.Cu) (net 7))
 (segment (start 163.322 98.8695) (end 161.8615 98.8695) (width 0.25) (layer F.Cu) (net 7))
 (segment (start 161.29 94.214) (end 163.068 92.436) (width 0.25) (layer F.Cu) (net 7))
 (segment (start 161.29 98.298) (end 161.29 94.214) (width 0.25) (layer F.Cu) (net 7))
 (segment (start 161.8615 98.8695) (end 161.29 98.298) (width 0.25) (layer F.Cu) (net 7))
 (segment (start 163.068 92.436) (end 165.12 92.436) (width 0.25) (layer F.Cu) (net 7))
 (segment (start 165.12 92.436) (end 165.63086 91.92514) (width 0.25) (layer F.Cu) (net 7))
 (segment (start 165.63086 91.92514) (end 166.878 91.92514) (width 0.25) (layer F.Cu) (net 7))
 (segment (start 163.322 98.8695) (end 166.6875 98.8695) (width 0.25) (layer F.Cu) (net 7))
 (segment (start 168.148 100.33) (end 168.148 101.774) (width 0.25) (layer F.Cu) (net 7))
 (segment (start 166.6875 98.8695) (end 168.148 100.33) (width 0.25) (layer F.Cu) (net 7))
 (segment (start 163.322 95.6945) (end 170.3705 95.6945) (width 0.25) (layer F.Cu) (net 19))
 (segment (start 171.704 97.028) (end 174.498 97.028) (width 0.25) (layer F.Cu) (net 19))
 (segment (start 170.3705 95.6945) (end 171.704 97.028) (width 0.25) (layer F.Cu) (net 19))
 (segment (start 174.498 97.028) (end 178.736 97.028) (width 0.25) (layer F.Cu) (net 19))
 (segment (start 158.242 97.5995) (end 154.2415 97.5995) (width 0.25) (layer F.Cu) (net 10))
 (segment (start 153.416 96.774) (end 151.13 96.774) (width 0.25) (layer F.Cu) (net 10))
 (segment (start 154.2415 97.5995) (end 153.416 96.774) (width 0.25) (layer F.Cu) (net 10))
 (segment (start 151.13 96.774) (end 146.892 96.774) (width 0.25) (layer F.Cu) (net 10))
 (segment (start 151.13 91.694) (end 151.892 91.694) (width 0.25) (layer F.Cu) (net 9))
 (segment (start 151.892 91.694) (end 156.5275 96.3295) (width 0.25) (layer F.Cu) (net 9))
 (segment (start 156.5275 96.3295) (end 158.242 96.3295) (width 0.25) (layer F.Cu) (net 9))
 (segment (start 151.13 91.694) (end 146.892 91.694) (width 0.25) (layer F.Cu) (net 9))
 (segment (start 158.242 100.7745) (end 157.2895 100.7745) (width 0.25) (layer F.Cu) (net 14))
 (segment (start 153.924 106.68) (end 151.13 109.474) (width 0.25) (layer F.Cu) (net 14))
 (segment (start 153.924 104.14) (end 153.924 106.68) (width 0.25) (layer F.Cu) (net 14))
 (segment (start 157.2895 100.7745) (end 153.924 104.14) (width 0.25) (layer F.Cu) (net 14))
 (segment (start 151.13 109.474) (end 146.892 109.474) (width 0.25) (layer F.Cu) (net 14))
 (segment (start 158.242 95.6945) (end 157.6705 95.6945) (width 0.25) (layer F.Cu) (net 8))
 (segment (start 157.6705 95.6945) (end 151.13 89.154) (width 0.25) (layer F.Cu) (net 8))
 (segment (start 151.13 89.154) (end 146.892 89.154) (width 0.25) (layer F.Cu) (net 8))
 (segment (start 158.242 99.5045) (end 156.0195 99.5045) (width 0.25) (layer F.Cu) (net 12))
 (segment (start 156.0195 99.5045) (end 151.13 104.394) (width 0.25) (layer F.Cu) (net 12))
 (segment (start 151.13 104.394) (end 146.892 104.394) (width 0.25) (layer F.Cu) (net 12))
 (segment (start 158.242 100.1395) (end 156.6545 100.1395) (width 0.25) (layer F.Cu) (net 13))
 (segment (start 152.908 105.156) (end 151.13 106.934) (width 0.25) (layer F.Cu) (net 13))
 (segment (start 152.908 103.886) (end 152.908 105.156) (width 0.25) (layer F.Cu) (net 13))
 (segment (start 156.6545 100.1395) (end 152.908 103.886) (width 0.25) (layer F.Cu) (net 13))
 (segment (start 146.892 106.934) (end 151.13 106.934) (width 0.25) (layer F.Cu) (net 13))
 (segment (start 158.242 98.2345) (end 155.2575 98.2345) (width 0.25) (layer F.Cu) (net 11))
 (segment (start 154.178 99.314) (end 151.13 99.314) (width 0.25) (layer F.Cu) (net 11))
 (segment (start 155.2575 98.2345) (end 154.178 99.314) (width 0.25) (layer F.Cu) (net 11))
 (segment (start 146.892 99.314) (end 151.13 99.314) (width 0.25) (layer F.Cu) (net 11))
 (segment (start 163.322 96.9645) (end 168.0845 96.9645) (width 0.25) (layer F.Cu) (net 17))
 (segment (start 173.228 102.108) (end 174.498 102.108) (width 0.25) (layer F.Cu) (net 17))
 (segment (start 168.0845 96.9645) (end 173.228 102.108) (width 0.25) (layer F.Cu) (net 17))
 (segment (start 174.498 102.108) (end 178.736 102.108) (width 0.25) (layer F.Cu) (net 17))
 (segment (start 163.322 97.5995) (end 167.4495 97.5995) (width 0.25) (layer F.Cu) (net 16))
 (segment (start 167.4495 97.5995) (end 174.498 104.648) (width 0.25) (layer F.Cu) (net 16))
 (segment (start 178.736 104.648) (end 174.498 104.648) (width 0.25) (layer F.Cu) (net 16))
 (segment (start 158.242 101.4095) (end 158.1785 101.4095) (width 0.25) (layer F.Cu) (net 15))
 (segment (start 158.1785 101.4095) (end 154.94 104.648) (width 0.25) (layer F.Cu) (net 15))
 (segment (start 154.94 104.648) (end 154.94 108.204) (width 0.25) (layer F.Cu) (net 15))
 (segment (start 154.94 108.204) (end 151.13 112.014) (width 0.25) (layer F.Cu) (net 15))
 (segment (start 146.892 112.014) (end 151.13 112.014) (width 0.25) (layer F.Cu) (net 15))
 (segment (start 163.322 96.3295) (end 169.7355 96.3295) (width 0.25) (layer F.Cu) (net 18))
 (segment (start 172.974 99.568) (end 174.498 99.568) (width 0.25) (layer F.Cu) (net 18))
 (segment (start 169.7355 96.3295) (end 172.974 99.568) (width 0.25) (layer F.Cu) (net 18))
 (segment (start 174.498 99.568) (end 178.736 99.568) (width 0.25) (layer F.Cu) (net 18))
 (segment (start 163.322 100.7745) (end 161.8615 100.7745) (width 0.25) (layer F.Cu) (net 20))
 (segment (start 159.766 105.41) (end 159.766 107.362) (width 0.25) (layer F.Cu) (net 20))
 (segment (start 161.036 104.14) (end 159.766 105.41) (width 0.25) (layer F.Cu) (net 20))
 (segment (start 161.036 101.6) (end 161.036 104.14) (width 0.25) (layer F.Cu) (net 20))
 (segment (start 161.8615 100.7745) (end 161.036 101.6) (width 0.25) (layer F.Cu) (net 20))
 (segment (start 162.56 107.362) (end 162.56 103.378) (width 0.25) (layer F.Cu) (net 21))
 (segment (start 163.322 102.616) (end 163.322 101.4095) (width 0.25) (layer F.Cu) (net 21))
 (segment (start 162.56 103.378) (end 163.322 102.616) (width 0.25) (layer F.Cu) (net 21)))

